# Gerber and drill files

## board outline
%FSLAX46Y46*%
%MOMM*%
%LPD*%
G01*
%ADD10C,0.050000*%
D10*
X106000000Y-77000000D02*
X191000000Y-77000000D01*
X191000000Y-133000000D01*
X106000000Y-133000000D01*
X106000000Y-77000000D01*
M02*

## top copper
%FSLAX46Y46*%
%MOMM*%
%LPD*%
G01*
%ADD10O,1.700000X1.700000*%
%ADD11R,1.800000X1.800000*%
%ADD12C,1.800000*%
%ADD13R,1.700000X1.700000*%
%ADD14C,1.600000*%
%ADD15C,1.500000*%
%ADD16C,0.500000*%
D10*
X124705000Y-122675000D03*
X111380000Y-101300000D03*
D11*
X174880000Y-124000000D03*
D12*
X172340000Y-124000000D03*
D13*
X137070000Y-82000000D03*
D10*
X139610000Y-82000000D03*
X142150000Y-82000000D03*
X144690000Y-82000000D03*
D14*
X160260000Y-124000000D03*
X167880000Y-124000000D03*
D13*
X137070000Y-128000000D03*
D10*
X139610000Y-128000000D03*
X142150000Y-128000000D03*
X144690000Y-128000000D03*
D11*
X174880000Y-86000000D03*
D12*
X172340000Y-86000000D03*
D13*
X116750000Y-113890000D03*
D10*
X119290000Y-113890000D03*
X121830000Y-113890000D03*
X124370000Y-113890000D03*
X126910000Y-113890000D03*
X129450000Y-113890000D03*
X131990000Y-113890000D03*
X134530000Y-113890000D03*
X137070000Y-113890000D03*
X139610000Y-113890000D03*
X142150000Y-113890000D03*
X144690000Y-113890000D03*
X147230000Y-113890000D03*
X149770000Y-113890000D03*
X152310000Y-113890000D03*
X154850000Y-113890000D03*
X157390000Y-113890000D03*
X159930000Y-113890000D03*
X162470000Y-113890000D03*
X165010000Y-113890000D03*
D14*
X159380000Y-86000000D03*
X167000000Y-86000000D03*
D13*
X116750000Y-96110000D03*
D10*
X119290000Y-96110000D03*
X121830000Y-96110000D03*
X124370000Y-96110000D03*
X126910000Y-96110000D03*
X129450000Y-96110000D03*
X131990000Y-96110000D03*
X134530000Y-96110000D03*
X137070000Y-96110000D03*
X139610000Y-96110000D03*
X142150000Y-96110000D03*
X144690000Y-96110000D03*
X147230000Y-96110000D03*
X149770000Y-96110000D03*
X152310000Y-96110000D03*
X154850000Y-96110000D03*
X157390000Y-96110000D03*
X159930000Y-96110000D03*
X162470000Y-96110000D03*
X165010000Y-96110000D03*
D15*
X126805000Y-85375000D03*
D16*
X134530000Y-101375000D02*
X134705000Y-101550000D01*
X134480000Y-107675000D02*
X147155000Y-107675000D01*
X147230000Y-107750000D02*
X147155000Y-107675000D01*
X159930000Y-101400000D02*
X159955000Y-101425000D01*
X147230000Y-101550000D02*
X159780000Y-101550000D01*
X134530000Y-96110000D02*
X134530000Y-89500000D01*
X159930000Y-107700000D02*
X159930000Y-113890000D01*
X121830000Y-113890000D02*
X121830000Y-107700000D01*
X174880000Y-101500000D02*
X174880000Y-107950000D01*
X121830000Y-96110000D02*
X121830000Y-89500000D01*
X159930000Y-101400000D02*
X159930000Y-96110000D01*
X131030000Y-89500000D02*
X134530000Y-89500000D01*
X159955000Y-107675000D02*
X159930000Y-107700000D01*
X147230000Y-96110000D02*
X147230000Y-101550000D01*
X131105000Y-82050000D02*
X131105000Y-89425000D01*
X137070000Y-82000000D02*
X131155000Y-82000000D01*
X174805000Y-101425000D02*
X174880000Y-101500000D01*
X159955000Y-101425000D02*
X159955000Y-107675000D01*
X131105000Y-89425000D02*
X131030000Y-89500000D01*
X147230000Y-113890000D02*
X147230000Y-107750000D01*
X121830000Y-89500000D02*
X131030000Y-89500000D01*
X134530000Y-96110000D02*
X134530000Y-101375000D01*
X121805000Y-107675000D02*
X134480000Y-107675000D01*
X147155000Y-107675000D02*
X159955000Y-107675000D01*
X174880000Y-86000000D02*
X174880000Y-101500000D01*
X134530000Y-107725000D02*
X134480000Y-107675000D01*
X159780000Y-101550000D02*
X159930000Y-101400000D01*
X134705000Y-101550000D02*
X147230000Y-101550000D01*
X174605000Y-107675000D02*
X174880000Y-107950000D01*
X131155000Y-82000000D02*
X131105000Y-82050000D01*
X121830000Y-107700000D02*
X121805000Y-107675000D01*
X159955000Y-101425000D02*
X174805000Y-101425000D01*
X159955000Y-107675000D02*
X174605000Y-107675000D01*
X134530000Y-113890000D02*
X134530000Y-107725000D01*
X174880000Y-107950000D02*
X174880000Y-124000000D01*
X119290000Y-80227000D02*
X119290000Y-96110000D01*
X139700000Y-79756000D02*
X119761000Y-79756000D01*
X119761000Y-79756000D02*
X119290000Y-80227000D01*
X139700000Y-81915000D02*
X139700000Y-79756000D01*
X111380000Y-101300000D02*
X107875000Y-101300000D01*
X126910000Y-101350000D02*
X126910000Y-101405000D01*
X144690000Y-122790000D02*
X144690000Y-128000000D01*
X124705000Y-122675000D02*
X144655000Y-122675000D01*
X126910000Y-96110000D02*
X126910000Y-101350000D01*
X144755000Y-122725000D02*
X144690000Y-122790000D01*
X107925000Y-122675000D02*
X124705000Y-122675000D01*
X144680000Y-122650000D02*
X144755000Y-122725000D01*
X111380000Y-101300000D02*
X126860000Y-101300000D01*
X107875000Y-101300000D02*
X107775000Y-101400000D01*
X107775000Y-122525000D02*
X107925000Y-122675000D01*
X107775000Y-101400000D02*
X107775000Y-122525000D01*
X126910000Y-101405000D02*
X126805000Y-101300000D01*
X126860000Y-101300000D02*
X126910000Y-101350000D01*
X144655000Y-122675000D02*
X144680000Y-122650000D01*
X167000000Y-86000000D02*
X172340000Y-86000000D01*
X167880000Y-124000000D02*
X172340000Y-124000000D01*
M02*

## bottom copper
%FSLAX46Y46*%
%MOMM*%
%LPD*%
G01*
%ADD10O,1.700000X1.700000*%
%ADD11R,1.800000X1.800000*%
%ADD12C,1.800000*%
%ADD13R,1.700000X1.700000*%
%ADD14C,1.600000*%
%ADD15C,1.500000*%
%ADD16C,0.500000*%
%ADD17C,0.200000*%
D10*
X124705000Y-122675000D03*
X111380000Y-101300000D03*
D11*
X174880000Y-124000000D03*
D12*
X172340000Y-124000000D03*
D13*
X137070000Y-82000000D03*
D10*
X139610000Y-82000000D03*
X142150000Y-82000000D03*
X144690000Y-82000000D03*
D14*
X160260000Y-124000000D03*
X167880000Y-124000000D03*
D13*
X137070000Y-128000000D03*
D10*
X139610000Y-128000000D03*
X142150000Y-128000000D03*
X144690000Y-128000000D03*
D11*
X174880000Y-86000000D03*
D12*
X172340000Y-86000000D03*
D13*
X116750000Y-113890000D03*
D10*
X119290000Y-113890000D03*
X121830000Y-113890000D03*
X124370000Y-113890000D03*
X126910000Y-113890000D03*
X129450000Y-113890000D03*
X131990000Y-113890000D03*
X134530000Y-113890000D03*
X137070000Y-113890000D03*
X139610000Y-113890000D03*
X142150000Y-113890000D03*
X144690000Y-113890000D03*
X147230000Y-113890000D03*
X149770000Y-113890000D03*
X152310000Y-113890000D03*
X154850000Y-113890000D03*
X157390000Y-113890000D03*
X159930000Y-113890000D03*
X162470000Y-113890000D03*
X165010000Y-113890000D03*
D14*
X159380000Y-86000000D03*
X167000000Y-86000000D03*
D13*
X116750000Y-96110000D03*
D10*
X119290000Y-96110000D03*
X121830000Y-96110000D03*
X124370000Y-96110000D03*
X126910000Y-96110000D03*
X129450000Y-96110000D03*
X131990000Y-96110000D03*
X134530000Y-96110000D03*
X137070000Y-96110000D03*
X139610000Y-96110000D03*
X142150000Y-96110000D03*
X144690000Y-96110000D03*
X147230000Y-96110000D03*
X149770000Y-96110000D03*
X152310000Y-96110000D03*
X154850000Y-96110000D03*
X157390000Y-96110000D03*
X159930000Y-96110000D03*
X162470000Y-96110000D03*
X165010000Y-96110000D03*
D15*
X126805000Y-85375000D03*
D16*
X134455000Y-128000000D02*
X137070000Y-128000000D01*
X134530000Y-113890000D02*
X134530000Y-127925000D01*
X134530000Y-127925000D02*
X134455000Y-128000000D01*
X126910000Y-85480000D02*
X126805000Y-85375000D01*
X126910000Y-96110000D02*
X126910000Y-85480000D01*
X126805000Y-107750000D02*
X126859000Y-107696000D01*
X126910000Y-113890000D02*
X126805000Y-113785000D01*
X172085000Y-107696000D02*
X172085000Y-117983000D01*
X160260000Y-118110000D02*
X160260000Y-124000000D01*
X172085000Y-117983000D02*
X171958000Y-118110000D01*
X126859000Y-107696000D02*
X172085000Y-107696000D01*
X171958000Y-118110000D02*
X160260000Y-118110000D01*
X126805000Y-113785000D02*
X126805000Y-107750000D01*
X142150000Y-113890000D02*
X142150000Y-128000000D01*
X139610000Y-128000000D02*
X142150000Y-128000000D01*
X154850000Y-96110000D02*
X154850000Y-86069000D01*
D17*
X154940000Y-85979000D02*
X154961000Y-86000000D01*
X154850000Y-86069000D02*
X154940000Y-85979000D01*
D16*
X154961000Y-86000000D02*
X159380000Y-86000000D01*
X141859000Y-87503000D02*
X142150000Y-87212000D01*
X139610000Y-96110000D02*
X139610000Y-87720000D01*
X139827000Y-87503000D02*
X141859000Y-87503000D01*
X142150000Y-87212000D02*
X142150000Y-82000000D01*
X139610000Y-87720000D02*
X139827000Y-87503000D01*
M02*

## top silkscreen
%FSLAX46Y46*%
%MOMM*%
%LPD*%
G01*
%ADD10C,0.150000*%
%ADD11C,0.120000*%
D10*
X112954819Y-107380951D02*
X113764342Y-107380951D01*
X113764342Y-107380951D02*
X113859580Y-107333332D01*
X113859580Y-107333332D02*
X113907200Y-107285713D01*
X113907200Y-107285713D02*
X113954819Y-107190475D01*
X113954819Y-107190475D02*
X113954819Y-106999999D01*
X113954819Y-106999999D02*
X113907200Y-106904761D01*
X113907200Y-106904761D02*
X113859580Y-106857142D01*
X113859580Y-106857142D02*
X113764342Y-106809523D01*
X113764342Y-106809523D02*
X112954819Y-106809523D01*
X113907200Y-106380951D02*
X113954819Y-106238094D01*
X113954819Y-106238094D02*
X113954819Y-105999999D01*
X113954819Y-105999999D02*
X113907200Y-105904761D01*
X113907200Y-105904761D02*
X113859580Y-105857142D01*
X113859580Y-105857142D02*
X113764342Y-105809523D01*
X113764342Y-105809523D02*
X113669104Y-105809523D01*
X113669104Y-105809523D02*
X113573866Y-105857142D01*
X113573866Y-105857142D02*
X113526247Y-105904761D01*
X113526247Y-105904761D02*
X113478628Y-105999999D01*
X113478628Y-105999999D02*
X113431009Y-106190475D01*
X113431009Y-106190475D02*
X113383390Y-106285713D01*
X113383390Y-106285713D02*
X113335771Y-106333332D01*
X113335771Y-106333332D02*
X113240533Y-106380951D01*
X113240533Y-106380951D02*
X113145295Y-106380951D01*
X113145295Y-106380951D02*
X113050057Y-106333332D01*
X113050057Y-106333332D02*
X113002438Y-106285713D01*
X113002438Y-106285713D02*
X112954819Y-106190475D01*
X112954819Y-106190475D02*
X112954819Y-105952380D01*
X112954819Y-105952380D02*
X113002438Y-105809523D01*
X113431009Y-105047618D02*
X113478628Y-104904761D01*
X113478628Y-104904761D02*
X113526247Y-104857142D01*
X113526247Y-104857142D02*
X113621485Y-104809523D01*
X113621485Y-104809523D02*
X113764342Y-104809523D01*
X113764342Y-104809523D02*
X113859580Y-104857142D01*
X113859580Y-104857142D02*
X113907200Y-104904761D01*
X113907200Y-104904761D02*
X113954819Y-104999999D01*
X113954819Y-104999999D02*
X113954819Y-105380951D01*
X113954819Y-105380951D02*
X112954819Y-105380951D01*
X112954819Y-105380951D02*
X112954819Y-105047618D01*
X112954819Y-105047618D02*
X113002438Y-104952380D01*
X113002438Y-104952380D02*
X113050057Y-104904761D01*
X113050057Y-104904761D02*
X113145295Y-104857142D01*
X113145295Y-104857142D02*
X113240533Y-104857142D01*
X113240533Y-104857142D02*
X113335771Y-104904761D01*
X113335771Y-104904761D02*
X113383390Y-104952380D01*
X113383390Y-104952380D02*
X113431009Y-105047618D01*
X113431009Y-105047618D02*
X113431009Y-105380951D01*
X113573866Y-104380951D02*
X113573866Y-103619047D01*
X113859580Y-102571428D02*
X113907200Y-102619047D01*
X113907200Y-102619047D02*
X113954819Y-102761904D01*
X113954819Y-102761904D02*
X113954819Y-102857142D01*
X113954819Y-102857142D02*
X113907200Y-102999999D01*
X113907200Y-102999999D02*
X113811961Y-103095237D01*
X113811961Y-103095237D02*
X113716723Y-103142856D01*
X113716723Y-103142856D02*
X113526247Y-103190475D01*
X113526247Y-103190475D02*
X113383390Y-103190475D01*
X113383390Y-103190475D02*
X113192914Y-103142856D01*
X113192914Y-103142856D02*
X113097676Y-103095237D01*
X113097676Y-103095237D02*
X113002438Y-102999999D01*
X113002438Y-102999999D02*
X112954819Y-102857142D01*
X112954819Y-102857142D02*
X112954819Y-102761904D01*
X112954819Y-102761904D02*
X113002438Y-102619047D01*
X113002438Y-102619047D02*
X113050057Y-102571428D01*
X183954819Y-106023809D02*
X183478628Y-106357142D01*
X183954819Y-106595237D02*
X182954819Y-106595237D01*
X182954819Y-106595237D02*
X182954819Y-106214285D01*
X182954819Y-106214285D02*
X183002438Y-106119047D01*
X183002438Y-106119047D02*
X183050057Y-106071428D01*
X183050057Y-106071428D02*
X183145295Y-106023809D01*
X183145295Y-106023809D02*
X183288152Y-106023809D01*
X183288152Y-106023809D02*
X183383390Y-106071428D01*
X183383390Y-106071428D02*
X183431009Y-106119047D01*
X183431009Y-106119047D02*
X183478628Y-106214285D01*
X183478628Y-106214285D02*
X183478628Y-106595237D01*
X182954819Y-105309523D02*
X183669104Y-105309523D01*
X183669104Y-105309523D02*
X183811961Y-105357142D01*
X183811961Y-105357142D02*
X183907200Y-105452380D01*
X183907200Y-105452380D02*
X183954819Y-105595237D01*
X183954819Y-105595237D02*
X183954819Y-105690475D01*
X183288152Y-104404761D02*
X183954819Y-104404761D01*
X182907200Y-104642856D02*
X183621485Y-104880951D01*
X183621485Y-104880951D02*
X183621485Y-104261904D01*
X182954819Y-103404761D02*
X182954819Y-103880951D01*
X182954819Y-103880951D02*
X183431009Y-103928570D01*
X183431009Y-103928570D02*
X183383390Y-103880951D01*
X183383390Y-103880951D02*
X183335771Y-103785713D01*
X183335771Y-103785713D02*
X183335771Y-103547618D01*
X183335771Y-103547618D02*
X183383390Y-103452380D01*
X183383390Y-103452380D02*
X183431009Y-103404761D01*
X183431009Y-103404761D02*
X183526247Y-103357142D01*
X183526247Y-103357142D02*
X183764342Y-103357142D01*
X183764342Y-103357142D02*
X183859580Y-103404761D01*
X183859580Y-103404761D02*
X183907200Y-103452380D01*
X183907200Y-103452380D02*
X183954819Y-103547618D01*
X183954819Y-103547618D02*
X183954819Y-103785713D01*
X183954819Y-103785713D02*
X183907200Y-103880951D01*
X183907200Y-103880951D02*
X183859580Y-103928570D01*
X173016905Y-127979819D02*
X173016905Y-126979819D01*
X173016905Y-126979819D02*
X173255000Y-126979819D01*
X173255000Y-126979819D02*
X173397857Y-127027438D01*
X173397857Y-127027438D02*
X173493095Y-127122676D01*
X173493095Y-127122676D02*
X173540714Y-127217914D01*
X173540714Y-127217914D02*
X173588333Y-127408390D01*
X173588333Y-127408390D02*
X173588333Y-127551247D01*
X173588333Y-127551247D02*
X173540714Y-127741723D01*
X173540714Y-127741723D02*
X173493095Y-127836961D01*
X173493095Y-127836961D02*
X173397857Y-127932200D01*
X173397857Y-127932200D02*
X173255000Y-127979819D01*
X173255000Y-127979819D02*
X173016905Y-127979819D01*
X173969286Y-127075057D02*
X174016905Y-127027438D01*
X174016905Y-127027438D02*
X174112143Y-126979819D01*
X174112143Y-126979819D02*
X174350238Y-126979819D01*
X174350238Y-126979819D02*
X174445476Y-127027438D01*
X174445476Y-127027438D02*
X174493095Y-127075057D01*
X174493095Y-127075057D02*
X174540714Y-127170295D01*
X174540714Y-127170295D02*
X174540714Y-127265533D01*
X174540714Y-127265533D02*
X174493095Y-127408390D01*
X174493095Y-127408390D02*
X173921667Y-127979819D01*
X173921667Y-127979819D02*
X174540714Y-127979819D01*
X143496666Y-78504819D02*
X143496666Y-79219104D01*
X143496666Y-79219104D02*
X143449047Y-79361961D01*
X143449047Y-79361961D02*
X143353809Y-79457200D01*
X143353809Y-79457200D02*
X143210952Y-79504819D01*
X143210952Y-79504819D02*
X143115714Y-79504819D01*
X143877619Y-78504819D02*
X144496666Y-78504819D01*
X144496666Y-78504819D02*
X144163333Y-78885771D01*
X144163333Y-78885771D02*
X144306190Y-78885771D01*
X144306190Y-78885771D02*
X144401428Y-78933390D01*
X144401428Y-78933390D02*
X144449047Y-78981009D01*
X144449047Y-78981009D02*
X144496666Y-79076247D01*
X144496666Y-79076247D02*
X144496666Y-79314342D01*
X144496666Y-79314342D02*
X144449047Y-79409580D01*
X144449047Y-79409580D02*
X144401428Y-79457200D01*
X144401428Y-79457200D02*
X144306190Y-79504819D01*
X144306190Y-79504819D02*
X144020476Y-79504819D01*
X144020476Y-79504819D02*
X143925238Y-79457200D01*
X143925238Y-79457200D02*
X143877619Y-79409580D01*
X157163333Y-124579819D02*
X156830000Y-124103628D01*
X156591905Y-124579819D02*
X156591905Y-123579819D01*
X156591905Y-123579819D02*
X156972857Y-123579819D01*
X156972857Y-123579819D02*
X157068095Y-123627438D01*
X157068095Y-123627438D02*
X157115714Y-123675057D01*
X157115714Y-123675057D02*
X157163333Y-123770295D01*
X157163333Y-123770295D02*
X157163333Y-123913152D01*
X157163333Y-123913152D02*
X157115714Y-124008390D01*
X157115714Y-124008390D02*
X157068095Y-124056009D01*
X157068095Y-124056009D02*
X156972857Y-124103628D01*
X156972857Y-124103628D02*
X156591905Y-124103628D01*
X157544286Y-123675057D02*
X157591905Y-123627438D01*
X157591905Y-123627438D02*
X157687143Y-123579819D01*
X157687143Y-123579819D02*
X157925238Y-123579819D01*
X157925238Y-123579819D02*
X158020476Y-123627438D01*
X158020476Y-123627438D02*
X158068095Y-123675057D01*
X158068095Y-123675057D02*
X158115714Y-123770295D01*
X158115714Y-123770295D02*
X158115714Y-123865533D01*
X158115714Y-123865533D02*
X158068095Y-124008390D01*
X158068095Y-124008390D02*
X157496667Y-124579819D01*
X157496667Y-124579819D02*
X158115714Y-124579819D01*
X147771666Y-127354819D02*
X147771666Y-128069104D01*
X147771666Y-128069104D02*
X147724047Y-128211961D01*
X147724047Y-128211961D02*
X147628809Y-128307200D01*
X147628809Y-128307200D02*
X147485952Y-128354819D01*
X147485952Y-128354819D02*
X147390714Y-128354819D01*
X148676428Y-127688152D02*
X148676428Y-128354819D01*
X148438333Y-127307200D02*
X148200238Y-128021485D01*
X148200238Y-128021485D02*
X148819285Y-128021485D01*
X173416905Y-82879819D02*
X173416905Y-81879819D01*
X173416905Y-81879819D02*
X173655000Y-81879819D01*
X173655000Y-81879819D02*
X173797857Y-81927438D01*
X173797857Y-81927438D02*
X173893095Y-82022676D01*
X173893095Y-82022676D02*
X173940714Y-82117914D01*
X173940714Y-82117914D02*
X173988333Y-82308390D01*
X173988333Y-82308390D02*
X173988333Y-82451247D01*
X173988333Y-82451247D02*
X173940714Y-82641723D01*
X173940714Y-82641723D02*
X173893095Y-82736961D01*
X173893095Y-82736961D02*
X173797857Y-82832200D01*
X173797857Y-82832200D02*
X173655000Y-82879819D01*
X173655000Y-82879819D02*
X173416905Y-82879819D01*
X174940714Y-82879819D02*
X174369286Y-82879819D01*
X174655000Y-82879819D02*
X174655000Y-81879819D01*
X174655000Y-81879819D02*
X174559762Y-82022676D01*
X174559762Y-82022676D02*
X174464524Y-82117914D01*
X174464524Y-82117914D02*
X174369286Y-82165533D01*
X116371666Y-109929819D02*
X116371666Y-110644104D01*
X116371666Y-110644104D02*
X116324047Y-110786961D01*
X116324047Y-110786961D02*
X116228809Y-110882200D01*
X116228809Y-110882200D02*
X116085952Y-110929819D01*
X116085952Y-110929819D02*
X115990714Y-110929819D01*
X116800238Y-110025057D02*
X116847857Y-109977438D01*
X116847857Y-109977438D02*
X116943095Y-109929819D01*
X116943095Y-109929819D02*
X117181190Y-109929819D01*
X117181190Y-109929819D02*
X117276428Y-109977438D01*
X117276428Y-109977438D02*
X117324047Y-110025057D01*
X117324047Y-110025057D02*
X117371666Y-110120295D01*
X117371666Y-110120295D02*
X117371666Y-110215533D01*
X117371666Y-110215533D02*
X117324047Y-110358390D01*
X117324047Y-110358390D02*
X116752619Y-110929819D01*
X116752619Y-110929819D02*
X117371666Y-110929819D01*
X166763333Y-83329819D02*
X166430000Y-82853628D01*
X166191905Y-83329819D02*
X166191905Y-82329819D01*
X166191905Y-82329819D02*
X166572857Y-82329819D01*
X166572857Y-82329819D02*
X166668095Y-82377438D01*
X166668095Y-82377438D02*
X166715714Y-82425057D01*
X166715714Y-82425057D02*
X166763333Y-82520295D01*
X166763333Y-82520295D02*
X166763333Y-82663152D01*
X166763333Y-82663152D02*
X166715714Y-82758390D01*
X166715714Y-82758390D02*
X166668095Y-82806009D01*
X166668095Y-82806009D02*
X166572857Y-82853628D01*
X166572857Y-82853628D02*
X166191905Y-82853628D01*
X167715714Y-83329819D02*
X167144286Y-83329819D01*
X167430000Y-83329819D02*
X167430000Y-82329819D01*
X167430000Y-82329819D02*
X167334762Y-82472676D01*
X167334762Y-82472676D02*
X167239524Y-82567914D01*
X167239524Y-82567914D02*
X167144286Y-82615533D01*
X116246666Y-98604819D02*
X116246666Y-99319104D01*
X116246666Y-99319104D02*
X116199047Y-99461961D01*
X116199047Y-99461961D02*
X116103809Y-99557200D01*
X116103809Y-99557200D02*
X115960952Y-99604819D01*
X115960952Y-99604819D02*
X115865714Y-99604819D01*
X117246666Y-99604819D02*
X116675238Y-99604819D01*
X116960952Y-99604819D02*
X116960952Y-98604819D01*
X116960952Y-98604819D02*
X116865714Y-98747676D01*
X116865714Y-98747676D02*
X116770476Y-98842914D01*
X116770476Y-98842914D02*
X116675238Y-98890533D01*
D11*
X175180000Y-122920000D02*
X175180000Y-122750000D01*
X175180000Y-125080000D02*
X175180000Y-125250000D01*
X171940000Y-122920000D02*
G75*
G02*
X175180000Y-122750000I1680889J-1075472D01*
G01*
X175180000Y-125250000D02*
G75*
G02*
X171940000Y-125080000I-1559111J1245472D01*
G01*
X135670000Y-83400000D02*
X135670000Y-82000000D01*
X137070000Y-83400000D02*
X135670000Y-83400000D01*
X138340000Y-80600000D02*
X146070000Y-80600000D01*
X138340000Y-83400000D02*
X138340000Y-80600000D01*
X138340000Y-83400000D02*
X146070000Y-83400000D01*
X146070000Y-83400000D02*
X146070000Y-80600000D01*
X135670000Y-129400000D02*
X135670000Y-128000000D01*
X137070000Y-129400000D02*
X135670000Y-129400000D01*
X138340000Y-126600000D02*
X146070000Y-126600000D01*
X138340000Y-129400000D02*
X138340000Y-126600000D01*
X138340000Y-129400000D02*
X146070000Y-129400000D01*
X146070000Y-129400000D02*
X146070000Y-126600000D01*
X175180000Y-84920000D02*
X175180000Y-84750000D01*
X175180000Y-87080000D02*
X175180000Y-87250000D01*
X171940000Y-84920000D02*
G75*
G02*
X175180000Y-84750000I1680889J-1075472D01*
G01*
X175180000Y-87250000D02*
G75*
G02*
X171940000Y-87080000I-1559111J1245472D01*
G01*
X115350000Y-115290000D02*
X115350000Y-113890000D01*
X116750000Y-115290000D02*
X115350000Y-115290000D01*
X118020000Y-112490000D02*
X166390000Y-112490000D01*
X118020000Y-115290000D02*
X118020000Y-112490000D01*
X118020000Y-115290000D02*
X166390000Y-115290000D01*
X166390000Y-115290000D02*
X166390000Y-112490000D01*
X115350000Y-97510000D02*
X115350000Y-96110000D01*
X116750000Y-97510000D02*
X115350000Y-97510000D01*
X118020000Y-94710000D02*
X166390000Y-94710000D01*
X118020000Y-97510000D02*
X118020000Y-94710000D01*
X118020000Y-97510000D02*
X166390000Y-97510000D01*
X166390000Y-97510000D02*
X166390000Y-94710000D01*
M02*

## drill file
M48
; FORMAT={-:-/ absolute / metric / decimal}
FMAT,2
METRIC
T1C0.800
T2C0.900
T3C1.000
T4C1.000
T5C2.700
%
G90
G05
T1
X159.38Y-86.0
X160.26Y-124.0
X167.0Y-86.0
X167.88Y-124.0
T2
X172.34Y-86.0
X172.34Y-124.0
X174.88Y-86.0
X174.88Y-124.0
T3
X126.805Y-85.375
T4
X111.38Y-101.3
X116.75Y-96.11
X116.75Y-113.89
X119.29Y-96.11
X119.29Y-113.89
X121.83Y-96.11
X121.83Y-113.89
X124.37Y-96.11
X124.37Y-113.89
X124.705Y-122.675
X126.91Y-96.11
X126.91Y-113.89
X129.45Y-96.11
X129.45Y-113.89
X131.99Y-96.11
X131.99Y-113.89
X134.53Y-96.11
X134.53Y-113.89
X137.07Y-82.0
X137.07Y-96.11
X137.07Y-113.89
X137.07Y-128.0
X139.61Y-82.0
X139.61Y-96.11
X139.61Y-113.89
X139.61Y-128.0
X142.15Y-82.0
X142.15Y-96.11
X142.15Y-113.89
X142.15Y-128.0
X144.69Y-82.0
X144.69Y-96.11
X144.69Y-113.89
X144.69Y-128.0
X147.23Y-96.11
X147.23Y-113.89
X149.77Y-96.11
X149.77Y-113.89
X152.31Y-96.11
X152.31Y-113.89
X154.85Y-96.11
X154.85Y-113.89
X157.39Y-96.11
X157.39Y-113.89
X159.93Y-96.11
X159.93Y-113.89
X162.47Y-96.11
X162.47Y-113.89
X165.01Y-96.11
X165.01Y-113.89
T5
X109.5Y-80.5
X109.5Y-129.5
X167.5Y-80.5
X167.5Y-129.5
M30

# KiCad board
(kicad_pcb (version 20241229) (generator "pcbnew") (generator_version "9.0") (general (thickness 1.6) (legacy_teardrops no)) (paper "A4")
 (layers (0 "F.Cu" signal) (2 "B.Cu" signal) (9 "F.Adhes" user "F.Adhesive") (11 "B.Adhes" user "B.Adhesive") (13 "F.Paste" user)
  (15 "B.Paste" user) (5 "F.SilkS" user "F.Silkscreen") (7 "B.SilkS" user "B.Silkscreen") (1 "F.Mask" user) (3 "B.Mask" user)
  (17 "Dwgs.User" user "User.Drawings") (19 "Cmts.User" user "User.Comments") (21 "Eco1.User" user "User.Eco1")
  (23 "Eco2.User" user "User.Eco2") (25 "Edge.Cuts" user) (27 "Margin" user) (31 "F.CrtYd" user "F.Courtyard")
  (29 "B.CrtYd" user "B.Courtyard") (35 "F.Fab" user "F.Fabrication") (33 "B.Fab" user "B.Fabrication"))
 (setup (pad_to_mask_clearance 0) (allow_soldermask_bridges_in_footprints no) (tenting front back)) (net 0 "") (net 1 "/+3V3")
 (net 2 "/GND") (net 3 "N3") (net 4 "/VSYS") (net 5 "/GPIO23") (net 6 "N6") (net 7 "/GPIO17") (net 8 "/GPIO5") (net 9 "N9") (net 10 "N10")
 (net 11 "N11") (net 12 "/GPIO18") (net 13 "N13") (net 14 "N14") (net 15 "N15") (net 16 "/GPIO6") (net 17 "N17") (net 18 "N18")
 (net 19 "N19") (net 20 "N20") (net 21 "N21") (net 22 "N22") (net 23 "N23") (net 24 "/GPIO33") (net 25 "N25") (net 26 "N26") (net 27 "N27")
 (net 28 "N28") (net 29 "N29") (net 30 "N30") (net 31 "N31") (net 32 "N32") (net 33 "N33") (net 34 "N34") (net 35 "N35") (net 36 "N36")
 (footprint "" (layer "F.Cu") (at 124.705 122.675)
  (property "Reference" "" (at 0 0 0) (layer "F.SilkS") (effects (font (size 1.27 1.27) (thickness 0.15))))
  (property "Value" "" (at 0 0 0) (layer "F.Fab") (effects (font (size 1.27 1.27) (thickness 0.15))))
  (pad "4" thru_hole oval (at 0 0) (size 1.7 1.7) (drill 1) (layers "*.Cu" "*.Mask") (remove_unused_layers no) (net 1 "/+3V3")))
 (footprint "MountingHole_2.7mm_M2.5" (layer "F.Cu") (at 109.5 129.5)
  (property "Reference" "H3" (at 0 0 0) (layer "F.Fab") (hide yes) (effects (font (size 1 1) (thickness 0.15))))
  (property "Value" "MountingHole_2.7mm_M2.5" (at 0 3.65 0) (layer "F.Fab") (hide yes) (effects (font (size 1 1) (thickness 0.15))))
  (pad "" np_thru_hole circle (at 0 0) (size 2.7 2.7) (drill 2.7) (layers "*.Cu" "*.Mask")))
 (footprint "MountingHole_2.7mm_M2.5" (layer "F.Cu") (at 167.5 129.5)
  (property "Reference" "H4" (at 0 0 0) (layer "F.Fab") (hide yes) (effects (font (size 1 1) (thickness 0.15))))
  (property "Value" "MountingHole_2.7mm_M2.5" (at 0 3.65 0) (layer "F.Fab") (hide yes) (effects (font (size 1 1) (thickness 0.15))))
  (pad "" np_thru_hole circle (at 0 0) (size 2.7 2.7) (drill 2.7) (layers "*.Cu" "*.Mask")))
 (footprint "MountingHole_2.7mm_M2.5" (layer "F.Cu") (at 167.5 80.5)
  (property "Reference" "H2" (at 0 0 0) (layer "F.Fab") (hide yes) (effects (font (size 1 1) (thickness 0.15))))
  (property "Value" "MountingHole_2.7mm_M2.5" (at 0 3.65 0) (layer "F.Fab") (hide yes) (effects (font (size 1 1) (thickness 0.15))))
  (pad "" np_thru_hole circle (at 0 0) (size 2.7 2.7) (drill 2.7) (layers "*.Cu" "*.Mask")))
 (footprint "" (layer "F.Cu") (at 111.38 101.3)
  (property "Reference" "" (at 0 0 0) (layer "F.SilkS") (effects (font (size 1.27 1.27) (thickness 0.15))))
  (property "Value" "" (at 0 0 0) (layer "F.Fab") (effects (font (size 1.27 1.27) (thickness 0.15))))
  (pad "4" thru_hole oval (at 0 0) (size 1.7 1.7) (drill 1) (layers "*.Cu" "*.Mask") (remove_unused_layers no) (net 1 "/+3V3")))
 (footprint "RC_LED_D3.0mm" (layer "F.Cu") (at 174.88 124 180)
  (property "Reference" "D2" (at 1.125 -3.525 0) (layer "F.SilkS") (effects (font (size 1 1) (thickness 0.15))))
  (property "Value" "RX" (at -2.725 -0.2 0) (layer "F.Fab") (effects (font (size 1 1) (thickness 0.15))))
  (fp_line (start -0.3 1.08) (end -0.3 1.25) (stroke (width 0.12) (type solid)) (layer "F.SilkS"))
  (fp_line (start -0.3 -1.08) (end -0.3 -1.25) (stroke (width 0.12) (type solid)) (layer "F.SilkS"))
  (fp_arc (start 2.94 1.08) (mid 1.27 2) (end -0.3 1.25) (stroke (width 0.12) (type solid)) (layer "F.SilkS"))
  (fp_arc (start -0.3 -1.25) (mid 1.27 -2) (end 2.94 -1.08) (stroke (width 0.12) (type solid)) (layer "F.SilkS"))
  (pad "1" thru_hole rect (at 0 0) (size 1.8 1.8) (drill 0.9) (layers "*.Cu" "*.Mask") (remove_unused_layers no) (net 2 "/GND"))
  (pad "2" thru_hole circle (at 2.54 0) (size 1.8 1.8) (drill 0.9) (layers "*.Cu" "*.Mask") (remove_unused_layers no) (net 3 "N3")))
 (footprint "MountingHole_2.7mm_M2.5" (layer "F.Cu") (at 109.5 80.5)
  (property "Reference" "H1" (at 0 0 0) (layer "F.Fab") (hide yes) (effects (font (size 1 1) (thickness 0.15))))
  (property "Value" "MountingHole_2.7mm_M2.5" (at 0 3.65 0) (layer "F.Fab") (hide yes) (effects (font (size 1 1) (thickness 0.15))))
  (pad "" np_thru_hole circle (at 0 0) (size 2.7 2.7) (drill 2.7) (layers "*.Cu" "*.Mask")))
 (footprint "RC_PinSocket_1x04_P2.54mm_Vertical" (layer "F.Cu") (at 137.07 82 90)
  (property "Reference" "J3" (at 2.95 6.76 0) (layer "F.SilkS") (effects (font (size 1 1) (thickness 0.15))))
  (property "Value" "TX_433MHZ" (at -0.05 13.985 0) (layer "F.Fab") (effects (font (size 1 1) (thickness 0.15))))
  (fp_line (start -1.4 -1.4) (end 0 -1.4) (stroke (width 0.12) (type solid)) (layer "F.SilkS"))
  (fp_line (start -1.4 0) (end -1.4 -1.4) (stroke (width 0.12) (type solid)) (layer "F.SilkS"))
  (fp_line (start 1.4 1.27) (end 1.4 9) (stroke (width 0.12) (type solid)) (layer "F.SilkS"))
  (fp_line (start -1.4 1.27) (end 1.4 1.27) (stroke (width 0.12) (type solid)) (layer "F.SilkS"))
  (fp_line (start -1.4 1.27) (end -1.4 9) (stroke (width 0.12) (type solid)) (layer "F.SilkS"))
  (fp_line (start -1.4 9) (end 1.4 9) (stroke (width 0.12) (type solid)) (layer "F.SilkS"))
  (pad "1" thru_hole rect (at 0 0) (size 1.7 1.7) (drill 1) (layers "*.Cu" "*.Mask") (remove_unused_layers no) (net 2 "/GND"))
  (pad "2" thru_hole oval (at 0 2.54) (size 1.7 1.7) (drill 1) (layers "*.Cu" "*.Mask") (remove_unused_layers no) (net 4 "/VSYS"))
  (pad "3" thru_hole oval (at 0 5.08) (size 1.7 1.7) (drill 1) (layers "*.Cu" "*.Mask") (remove_unused_layers no) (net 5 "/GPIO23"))
  (pad "4" thru_hole oval (at 0 7.62) (size 1.7 1.7) (drill 1) (layers "*.Cu" "*.Mask") (remove_unused_layers no) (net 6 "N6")))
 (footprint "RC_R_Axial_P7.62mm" (layer "F.Cu") (at 160.26 124)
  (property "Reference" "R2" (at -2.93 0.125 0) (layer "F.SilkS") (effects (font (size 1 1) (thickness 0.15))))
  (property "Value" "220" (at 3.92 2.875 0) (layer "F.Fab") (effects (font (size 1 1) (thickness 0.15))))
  (pad "1" thru_hole circle (at 0 0) (size 1.6 1.6) (drill 0.8) (layers "*.Cu" "*.Mask") (remove_unused_layers no) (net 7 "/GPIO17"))
  (pad "2" thru_hole circle (at 7.62 0) (size 1.6 1.6) (drill 0.8) (layers "*.Cu" "*.Mask") (remove_unused_layers no) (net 3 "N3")))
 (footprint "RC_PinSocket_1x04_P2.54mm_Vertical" (layer "F.Cu") (at 137.07 128 90)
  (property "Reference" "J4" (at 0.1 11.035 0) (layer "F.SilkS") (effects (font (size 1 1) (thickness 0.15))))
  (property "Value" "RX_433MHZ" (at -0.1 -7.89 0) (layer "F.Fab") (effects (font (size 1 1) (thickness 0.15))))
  (fp_line (start -1.4 -1.4) (end 0 -1.4) (stroke (width 0.12) (type solid)) (layer "F.SilkS"))
  (fp_line (start -1.4 0) (end -1.4 -1.4) (stroke (width 0.12) (type solid)) (layer "F.SilkS"))
  (fp_line (start 1.4 1.27) (end 1.4 9) (stroke (width 0.12) (type solid)) (layer "F.SilkS"))
  (fp_line (start -1.4 1.27) (end 1.4 1.27) (stroke (width 0.12) (type solid)) (layer "F.SilkS"))
  (fp_line (start -1.4 1.27) (end -1.4 9) (stroke (width 0.12) (type solid)) (layer "F.SilkS"))
  (fp_line (start -1.4 9) (end 1.4 9) (stroke (width 0.12) (type solid)) (layer "F.SilkS"))
  (pad "1" thru_hole rect (at 0 0) (size 1.7 1.7) (drill 1) (layers "*.Cu" "*.Mask") (remove_unused_layers no) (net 2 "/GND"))
  (pad "2" thru_hole oval (at 0 2.54) (size 1.7 1.7) (drill 1) (layers "*.Cu" "*.Mask") (remove_unused_layers no) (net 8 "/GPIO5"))
  (pad "3" thru_hole oval (at 0 5.08) (size 1.7 1.7) (drill 1) (layers "*.Cu" "*.Mask") (remove_unused_layers no) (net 8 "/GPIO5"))
  (pad "4" thru_hole oval (at 0 7.62) (size 1.7 1.7) (drill 1) (layers "*.Cu" "*.Mask") (remove_unused_layers no) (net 1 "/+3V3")))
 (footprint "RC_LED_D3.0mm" (layer "F.Cu") (at 174.88 86 180)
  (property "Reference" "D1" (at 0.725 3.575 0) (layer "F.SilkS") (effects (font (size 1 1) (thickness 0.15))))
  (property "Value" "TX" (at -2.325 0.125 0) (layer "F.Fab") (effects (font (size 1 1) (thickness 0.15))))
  (fp_line (start -0.3 1.08) (end -0.3 1.25) (stroke (width 0.12) (type solid)) (layer "F.SilkS"))
  (fp_line (start -0.3 -1.08) (end -0.3 -1.25) (stroke (width 0.12) (type solid)) (layer "F.SilkS"))
  (fp_arc (start 2.94 1.08) (mid 1.27 2) (end -0.3 1.25) (stroke (width 0.12) (type solid)) (layer "F.SilkS"))
  (fp_arc (start -0.3 -1.25) (mid 1.27 -2) (end 2.94 -1.08) (stroke (width 0.12) (type solid)) (layer "F.SilkS"))
  (pad "1" thru_hole rect (at 0 0) (size 1.8 1.8) (drill 0.9) (layers "*.Cu" "*.Mask") (remove_unused_layers no) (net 2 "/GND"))
  (pad "2" thru_hole circle (at 2.54 0) (size 1.8 1.8) (drill 0.9) (layers "*.Cu" "*.Mask") (remove_unused_layers no) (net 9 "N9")))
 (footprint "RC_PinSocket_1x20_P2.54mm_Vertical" (layer "F.Cu") (at 116.75 113.89 90)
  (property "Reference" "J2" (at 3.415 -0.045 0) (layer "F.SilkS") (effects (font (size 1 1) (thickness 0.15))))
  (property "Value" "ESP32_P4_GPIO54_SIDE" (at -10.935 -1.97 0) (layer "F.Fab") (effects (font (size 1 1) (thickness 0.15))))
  (fp_line (start -1.4 -1.4) (end 0 -1.4) (stroke (width 0.12) (type solid)) (layer "F.SilkS"))
  (fp_line (start -1.4 0) (end -1.4 -1.4) (stroke (width 0.12) (type solid)) (layer "F.SilkS"))
  (fp_line (start 1.4 1.27) (end 1.4 49.64) (stroke (width 0.12) (type solid)) (layer "F.SilkS"))
  (fp_line (start -1.4 1.27) (end 1.4 1.27) (stroke (width 0.12) (type solid)) (layer "F.SilkS"))
  (fp_line (start -1.4 1.27) (end -1.4 49.64) (stroke (width 0.12) (type solid)) (layer "F.SilkS"))
  (fp_line (start -1.4 49.64) (end 1.4 49.64) (stroke (width 0.12) (type solid)) (layer "F.SilkS"))
  (pad "1" thru_hole rect (at 0 0) (size 1.7 1.7) (drill 1) (layers "*.Cu" "*.Mask") (remove_unused_layers no) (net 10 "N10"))
  (pad "2" thru_hole oval (at 0 2.54) (size 1.7 1.7) (drill 1) (layers "*.Cu" "*.Mask") (remove_unused_layers no) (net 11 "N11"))
  (pad "3" thru_hole oval (at 0 5.08) (size 1.7 1.7) (drill 1) (layers "*.Cu" "*.Mask") (remove_unused_layers no) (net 2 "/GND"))
  (pad "4" thru_hole oval (at 0 7.62) (size 1.7 1.7) (drill 1) (layers "*.Cu" "*.Mask") (remove_unused_layers no) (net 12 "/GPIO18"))
  (pad "5" thru_hole oval (at 0 10.16) (size 1.7 1.7) (drill 1) (layers "*.Cu" "*.Mask") (remove_unused_layers no) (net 7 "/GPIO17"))
  (pad "6" thru_hole oval (at 0 12.7) (size 1.7 1.7) (drill 1) (layers "*.Cu" "*.Mask") (remove_unused_layers no) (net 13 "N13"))
  (pad "7" thru_hole oval (at 0 15.24) (size 1.7 1.7) (drill 1) (layers "*.Cu" "*.Mask") (remove_unused_layers no) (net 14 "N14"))
  (pad "8" thru_hole oval (at 0 17.78) (size 1.7 1.7) (drill 1) (layers "*.Cu" "*.Mask") (remove_unused_layers no) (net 2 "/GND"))
  (pad "9" thru_hole oval (at 0 20.32) (size 1.7 1.7) (drill 1) (layers "*.Cu" "*.Mask") (remove_unused_layers no) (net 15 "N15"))
  (pad "10" thru_hole oval (at 0 22.86) (size 1.7 1.7) (drill 1) (layers "*.Cu" "*.Mask") (remove_unused_layers no) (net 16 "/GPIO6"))
  (pad "11" thru_hole oval (at 0 25.4) (size 1.7 1.7) (drill 1) (layers "*.Cu" "*.Mask") (remove_unused_layers no) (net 8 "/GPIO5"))
  (pad "12" thru_hole oval (at 0 27.94) (size 1.7 1.7) (drill 1) (layers "*.Cu" "*.Mask") (remove_unused_layers no) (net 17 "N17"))
  (pad "13" thru_hole oval (at 0 30.48) (size 1.7 1.7) (drill 1) (layers "*.Cu" "*.Mask") (remove_unused_layers no) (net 2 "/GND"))
  (pad "14" thru_hole oval (at 0 33.02) (size 1.7 1.7) (drill 1) (layers "*.Cu" "*.Mask") (remove_unused_layers no) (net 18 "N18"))
  (pad "15" thru_hole oval (at 0 35.56) (size 1.7 1.7) (drill 1) (layers "*.Cu" "*.Mask") (remove_unused_layers no) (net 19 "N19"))
  (pad "16" thru_hole oval (at 0 38.1) (size 1.7 1.7) (drill 1) (layers "*.Cu" "*.Mask") (remove_unused_layers no) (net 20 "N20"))
  (pad "17" thru_hole oval (at 0 40.64) (size 1.7 1.7) (drill 1) (layers "*.Cu" "*.Mask") (remove_unused_layers no) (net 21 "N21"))
  (pad "18" thru_hole oval (at 0 43.18) (size 1.7 1.7) (drill 1) (layers "*.Cu" "*.Mask") (remove_unused_layers no) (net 2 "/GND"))
  (pad "19" thru_hole oval (at 0 45.72) (size 1.7 1.7) (drill 1) (layers "*.Cu" "*.Mask") (remove_unused_layers no) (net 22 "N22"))
  (pad "20" thru_hole oval (at 0 48.26) (size 1.7 1.7) (drill 1) (layers "*.Cu" "*.Mask") (remove_unused_layers no) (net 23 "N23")))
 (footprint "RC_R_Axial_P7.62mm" (layer "F.Cu") (at 159.38 86)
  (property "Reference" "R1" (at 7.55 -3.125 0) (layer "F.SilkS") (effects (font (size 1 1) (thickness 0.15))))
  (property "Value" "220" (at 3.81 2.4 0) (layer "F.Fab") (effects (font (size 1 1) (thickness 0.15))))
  (pad "1" thru_hole circle (at 0 0) (size 1.6 1.6) (drill 0.8) (layers "*.Cu" "*.Mask") (remove_unused_layers no) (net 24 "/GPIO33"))
  (pad "2" thru_hole circle (at 7.62 0) (size 1.6 1.6) (drill 0.8) (layers "*.Cu" "*.Mask") (remove_unused_layers no) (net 9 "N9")))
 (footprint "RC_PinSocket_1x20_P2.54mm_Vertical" (layer "F.Cu") (at 116.75 96.11 90)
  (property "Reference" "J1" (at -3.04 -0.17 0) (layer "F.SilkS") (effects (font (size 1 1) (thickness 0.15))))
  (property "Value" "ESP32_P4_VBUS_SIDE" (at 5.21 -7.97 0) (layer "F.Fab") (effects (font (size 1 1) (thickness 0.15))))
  (fp_line (start -1.4 -1.4) (end 0 -1.4) (stroke (width 0.12) (type solid)) (layer "F.SilkS"))
  (fp_line (start -1.4 0) (end -1.4 -1.4) (stroke (width 0.12) (type solid)) (layer "F.SilkS"))
  (fp_line (start 1.4 1.27) (end 1.4 49.64) (stroke (width 0.12) (type solid)) (layer "F.SilkS"))
  (fp_line (start -1.4 1.27) (end 1.4 1.27) (stroke (width 0.12) (type solid)) (layer "F.SilkS"))
  (fp_line (start -1.4 1.27) (end -1.4 49.64) (stroke (width 0.12) (type solid)) (layer "F.SilkS"))
  (fp_line (start -1.4 49.64) (end 1.4 49.64) (stroke (width 0.12) (type solid)) (layer "F.SilkS"))
  (pad "1" thru_hole rect (at 0 0) (size 1.7 1.7) (drill 1) (layers "*.Cu" "*.Mask") (remove_unused_layers no) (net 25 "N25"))
  (pad "2" thru_hole oval (at 0 2.54) (size 1.7 1.7) (drill 1) (layers "*.Cu" "*.Mask") (remove_unused_layers no) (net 4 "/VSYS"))
  (pad "3" thru_hole oval (at 0 5.08) (size 1.7 1.7) (drill 1) (layers "*.Cu" "*.Mask") (remove_unused_layers no) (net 2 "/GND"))
  (pad "4" thru_hole oval (at 0 7.62) (size 1.7 1.7) (drill 1) (layers "*.Cu" "*.Mask") (remove_unused_layers no) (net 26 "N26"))
  (pad "5" thru_hole oval (at 0 10.16) (size 1.7 1.7) (drill 1) (layers "*.Cu" "*.Mask") (remove_unused_layers no) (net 1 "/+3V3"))
  (pad "6" thru_hole oval (at 0 12.7) (size 1.7 1.7) (drill 1) (layers "*.Cu" "*.Mask") (remove_unused_layers no) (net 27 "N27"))
  (pad "7" thru_hole oval (at 0 15.24) (size 1.7 1.7) (drill 1) (layers "*.Cu" "*.Mask") (remove_unused_layers no) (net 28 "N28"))
  (pad "8" thru_hole oval (at 0 17.78) (size 1.7 1.7) (drill 1) (layers "*.Cu" "*.Mask") (remove_unused_layers no) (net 2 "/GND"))
  (pad "9" thru_hole oval (at 0 20.32) (size 1.7 1.7) (drill 1) (layers "*.Cu" "*.Mask") (remove_unused_layers no) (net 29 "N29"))
  (pad "10" thru_hole oval (at 0 22.86) (size 1.7 1.7) (drill 1) (layers "*.Cu" "*.Mask") (remove_unused_layers no) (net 5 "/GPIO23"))
  (pad "11" thru_hole oval (at 0 25.4) (size 1.7 1.7) (drill 1) (layers "*.Cu" "*.Mask") (remove_unused_layers no) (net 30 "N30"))
  (pad "12" thru_hole oval (at 0 27.94) (size 1.7 1.7) (drill 1) (layers "*.Cu" "*.Mask") (remove_unused_layers no) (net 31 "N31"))
  (pad "13" thru_hole oval (at 0 30.48) (size 1.7 1.7) (drill 1) (layers "*.Cu" "*.Mask") (remove_unused_layers no) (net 2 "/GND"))
  (pad "14" thru_hole oval (at 0 33.02) (size 1.7 1.7) (drill 1) (layers "*.Cu" "*.Mask") (remove_unused_layers no) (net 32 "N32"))
  (pad "15" thru_hole oval (at 0 35.56) (size 1.7 1.7) (drill 1) (layers "*.Cu" "*.Mask") (remove_unused_layers no) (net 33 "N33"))
  (pad "16" thru_hole oval (at 0 38.1) (size 1.7 1.7) (drill 1) (layers "*.Cu" "*.Mask") (remove_unused_layers no) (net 24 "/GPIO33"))
  (pad "17" thru_hole oval (at 0 40.64) (size 1.7 1.7) (drill 1) (layers "*.Cu" "*.Mask") (remove_unused_layers no) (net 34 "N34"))
  (pad "18" thru_hole oval (at 0 43.18) (size 1.7 1.7) (drill 1) (layers "*.Cu" "*.Mask") (remove_unused_layers no) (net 2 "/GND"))
  (pad "19" thru_hole oval (at 0 45.72) (size 1.7 1.7) (drill 1) (layers "*.Cu" "*.Mask") (remove_unused_layers no) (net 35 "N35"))
  (pad "20" thru_hole oval (at 0 48.26) (size 1.7 1.7) (drill 1) (layers "*.Cu" "*.Mask") (remove_unused_layers no) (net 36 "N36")))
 (gr_rect (start 106 77) (end 191 133) (stroke (width 0.05) (type solid)) (fill no) (layer "Edge.Cuts"))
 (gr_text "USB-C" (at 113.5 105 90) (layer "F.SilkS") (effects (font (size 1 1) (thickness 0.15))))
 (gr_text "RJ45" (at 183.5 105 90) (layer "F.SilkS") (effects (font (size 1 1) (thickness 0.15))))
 (segment (start 134.53 101.375) (end 134.705 101.55) (width 0.5) (layer "F.Cu") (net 2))
 (segment (start 134.48 107.675) (end 147.155 107.675) (width 0.5) (layer "F.Cu") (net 2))
 (segment (start 147.23 107.75) (end 147.155 107.675) (width 0.5) (layer "F.Cu") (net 2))
 (segment (start 159.93 101.4) (end 159.955 101.425) (width 0.5) (layer "F.Cu") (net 2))
 (segment (start 147.23 101.55) (end 159.78 101.55) (width 0.5) (layer "F.Cu") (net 2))
 (segment (start 134.53 96.11) (end 134.53 89.5) (width 0.5) (layer "F.Cu") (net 2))
 (segment (start 159.93 107.7) (end 159.93 113.89) (width 0.5) (layer "F.Cu") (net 2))
 (segment (start 121.83 113.89) (end 121.83 107.7) (width 0.5) (layer "F.Cu") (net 2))
 (segment (start 174.88 101.5) (end 174.88 107.95) (width 0.5) (layer "F.Cu") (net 2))
 (segment (start 121.83 96.11) (end 121.83 89.5) (width 0.5) (layer "F.Cu") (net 2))
 (segment (start 159.93 101.4) (end 159.93 96.11) (width 0.5) (layer "F.Cu") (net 2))
 (segment (start 131.03 89.5) (end 134.53 89.5) (width 0.5) (layer "F.Cu") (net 2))
 (segment (start 159.955 107.675) (end 159.93 107.7) (width 0.5) (layer "F.Cu") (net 2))
 (segment (start 147.23 96.11) (end 147.23 101.55) (width 0.5) (layer "F.Cu") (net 2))
 (segment (start 131.105 82.05) (end 131.105 89.425) (width 0.5) (layer "F.Cu") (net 2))
 (segment (start 137.07 82) (end 131.155 82) (width 0.5) (layer "F.Cu") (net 2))
 (segment (start 174.805 101.425) (end 174.88 101.5) (width 0.5) (layer "F.Cu") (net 2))
 (segment (start 159.955 101.425) (end 159.955 107.675) (width 0.5) (layer "F.Cu") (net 2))
 (segment (start 131.105 89.425) (end 131.03 89.5) (width 0.5) (layer "F.Cu") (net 2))
 (segment (start 147.23 113.89) (end 147.23 107.75) (width 0.5) (layer "F.Cu") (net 2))
 (segment (start 121.83 89.5) (end 131.03 89.5) (width 0.5) (layer "F.Cu") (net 2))
 (segment (start 134.53 96.11) (end 134.53 101.375) (width 0.5) (layer "F.Cu") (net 2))
 (segment (start 121.805 107.675) (end 134.48 107.675) (width 0.5) (layer "F.Cu") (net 2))
 (segment (start 147.155 107.675) (end 159.955 107.675) (width 0.5) (layer "F.Cu") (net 2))
 (segment (start 174.88 86) (end 174.88 101.5) (width 0.5) (layer "F.Cu") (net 2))
 (segment (start 134.53 107.725) (end 134.48 107.675) (width 0.5) (layer "F.Cu") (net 2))
 (segment (start 159.78 101.55) (end 159.93 101.4) (width 0.5) (layer "F.Cu") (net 2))
 (segment (start 134.705 101.55) (end 147.23 101.55) (width 0.5) (layer "F.Cu") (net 2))
 (segment (start 174.605 107.675) (end 174.88 107.95) (width 0.5) (layer "F.Cu") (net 2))
 (segment (start 131.155 82) (end 131.105 82.05) (width 0.5) (layer "F.Cu") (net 2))
 (segment (start 121.83 107.7) (end 121.805 107.675) (width 0.5) (layer "F.Cu") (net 2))
 (segment (start 159.955 101.425) (end 174.805 101.425) (width 0.5) (layer "F.Cu") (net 2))
 (segment (start 159.955 107.675) (end 174.605 107.675) (width 0.5) (layer "F.Cu") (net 2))
 (segment (start 134.53 113.89) (end 134.53 107.725) (width 0.5) (layer "F.Cu") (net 2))
 (segment (start 174.88 107.95) (end 174.88 124) (width 0.5) (layer "F.Cu") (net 2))
 (segment (start 134.455 128) (end 137.07 128) (width 0.5) (layer "B.Cu") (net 2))
 (segment (start 134.53 113.89) (end 134.53 127.925) (width 0.5) (layer "B.Cu") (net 2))
 (segment (start 134.53 127.925) (end 134.455 128) (width 0.5) (layer "B.Cu") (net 2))
 (segment (start 119.29 80.227) (end 119.29 96.11) (width 0.5) (layer "F.Cu") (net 4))
 (segment (start 139.7 79.756) (end 119.761 79.756) (width 0.5) (layer "F.Cu") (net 4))
 (segment (start 119.761 79.756) (end 119.29 80.227) (width 0.5) (layer "F.Cu") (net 4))
 (segment (start 139.7 81.915) (end 139.7 79.756) (width 0.5) (layer "F.Cu") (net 4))
 (segment (start 111.38 101.3) (end 107.875 101.3) (width 0.5) (layer "F.Cu") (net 1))
 (segment (start 126.91 101.35) (end 126.91 101.405) (width 0.5) (layer "F.Cu") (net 1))
 (segment (start 144.69 122.79) (end 144.69 128) (width 0.5) (layer "F.Cu") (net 1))
 (segment (start 124.705 122.675) (end 144.655 122.675) (width 0.5) (layer "F.Cu") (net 1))
 (segment (start 126.91 96.11) (end 126.91 101.35) (width 0.5) (layer "F.Cu") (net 1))
 (segment (start 144.755 122.725) (end 144.69 122.79) (width 0.5) (layer "F.Cu") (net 1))
 (segment (start 107.925 122.675) (end 124.705 122.675) (width 0.5) (layer "F.Cu") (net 1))
 (segment (start 144.68 122.65) (end 144.755 122.725) (width 0.5) (layer "F.Cu") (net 1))
 (segment (start 111.38 101.3) (end 126.86 101.3) (width 0.5) (layer "F.Cu") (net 1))
 (segment (start 107.875 101.3) (end 107.775 101.4) (width 0.5) (layer "F.Cu") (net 1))
 (segment (start 107.775 122.525) (end 107.925 122.675) (width 0.5) (layer "F.Cu") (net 1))
 (segment (start 107.775 101.4) (end 107.775 122.525) (width 0.5) (layer "F.Cu") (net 1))
 (segment (start 126.91 101.405) (end 126.805 101.3) (width 0.5) (layer "F.Cu") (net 1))
 (segment (start 126.86 101.3) (end 126.91 101.35) (width 0.5) (layer "F.Cu") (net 1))
 (segment (start 144.655 122.675) (end 144.68 122.65) (width 0.5) (layer "F.Cu") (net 1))
 (via (at 126.805 85.375) (size 1.5) (drill 1) (layers "F.Cu" "B.Cu") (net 1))
 (segment (start 126.91 85.48) (end 126.805 85.375) (width 0.5) (layer "B.Cu") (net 1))
 (segment (start 126.91 96.11) (end 126.91 85.48) (width 0.5) (layer "B.Cu") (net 1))
 (segment (start 167 86) (end 172.34 86) (width 0.5) (layer "F.Cu") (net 9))
 (segment (start 126.805 107.75) (end 126.859 107.696) (width 0.5) (layer "B.Cu") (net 7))
 (segment (start 126.91 113.89) (end 126.805 113.785) (width 0.5) (layer "B.Cu") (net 7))
 (segment (start 172.085 107.696) (end 172.085 117.983) (width 0.5) (layer "B.Cu") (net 7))
 (segment (start 160.26 118.11) (end 160.26 124) (width 0.5) (layer "B.Cu") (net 7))
 (segment (start 172.085 117.983) (end 171.958 118.11) (width 0.5) (layer "B.Cu") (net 7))
 (segment (start 126.859 107.696) (end 172.085 107.696) (width 0.5) (layer "B.Cu") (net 7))
 (segment (start 171.958 118.11) (end 160.26 118.11) (width 0.5) (layer "B.Cu") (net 7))
 (segment (start 126.805 113.785) (end 126.805 107.75) (width 0.5) (layer "B.Cu") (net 7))
 (segment (start 167.88 124) (end 172.34 124) (width 0.5) (layer "F.Cu") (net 3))
 (segment (start 142.15 113.89) (end 142.15 128) (width 0.5) (layer "B.Cu") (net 8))
 (segment (start 139.61 128) (end 142.15 128) (width 0.5) (layer "B.Cu") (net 8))
 (segment (start 154.85 96.11) (end 154.85 86.069) (width 0.5) (layer "B.Cu") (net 24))
 (segment (start 154.94 85.979) (end 154.961 86) (width 0.2) (layer "B.Cu") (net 24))
 (segment (start 154.85 86.069) (end 154.94 85.979) (width 0.2) (layer "B.Cu") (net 24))
 (segment (start 154.961 86) (end 159.38 86) (width 0.5) (layer "B.Cu") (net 24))
 (segment (start 141.859 87.503) (end 142.15 87.212) (width 0.5) (layer "B.Cu") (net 5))
 (segment (start 139.61 96.11) (end 139.61 87.72) (width 0.5) (layer "B.Cu") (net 5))
 (segment (start 139.827 87.503) (end 141.859 87.503) (width 0.5) (layer "B.Cu") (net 5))
 (segment (start 142.15 87.212) (end 142.15 82) (width 0.5) (layer "B.Cu") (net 5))
 (segment (start 139.61 87.72) (end 139.827 87.503) (width 0.5) (layer "B.Cu") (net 5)))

